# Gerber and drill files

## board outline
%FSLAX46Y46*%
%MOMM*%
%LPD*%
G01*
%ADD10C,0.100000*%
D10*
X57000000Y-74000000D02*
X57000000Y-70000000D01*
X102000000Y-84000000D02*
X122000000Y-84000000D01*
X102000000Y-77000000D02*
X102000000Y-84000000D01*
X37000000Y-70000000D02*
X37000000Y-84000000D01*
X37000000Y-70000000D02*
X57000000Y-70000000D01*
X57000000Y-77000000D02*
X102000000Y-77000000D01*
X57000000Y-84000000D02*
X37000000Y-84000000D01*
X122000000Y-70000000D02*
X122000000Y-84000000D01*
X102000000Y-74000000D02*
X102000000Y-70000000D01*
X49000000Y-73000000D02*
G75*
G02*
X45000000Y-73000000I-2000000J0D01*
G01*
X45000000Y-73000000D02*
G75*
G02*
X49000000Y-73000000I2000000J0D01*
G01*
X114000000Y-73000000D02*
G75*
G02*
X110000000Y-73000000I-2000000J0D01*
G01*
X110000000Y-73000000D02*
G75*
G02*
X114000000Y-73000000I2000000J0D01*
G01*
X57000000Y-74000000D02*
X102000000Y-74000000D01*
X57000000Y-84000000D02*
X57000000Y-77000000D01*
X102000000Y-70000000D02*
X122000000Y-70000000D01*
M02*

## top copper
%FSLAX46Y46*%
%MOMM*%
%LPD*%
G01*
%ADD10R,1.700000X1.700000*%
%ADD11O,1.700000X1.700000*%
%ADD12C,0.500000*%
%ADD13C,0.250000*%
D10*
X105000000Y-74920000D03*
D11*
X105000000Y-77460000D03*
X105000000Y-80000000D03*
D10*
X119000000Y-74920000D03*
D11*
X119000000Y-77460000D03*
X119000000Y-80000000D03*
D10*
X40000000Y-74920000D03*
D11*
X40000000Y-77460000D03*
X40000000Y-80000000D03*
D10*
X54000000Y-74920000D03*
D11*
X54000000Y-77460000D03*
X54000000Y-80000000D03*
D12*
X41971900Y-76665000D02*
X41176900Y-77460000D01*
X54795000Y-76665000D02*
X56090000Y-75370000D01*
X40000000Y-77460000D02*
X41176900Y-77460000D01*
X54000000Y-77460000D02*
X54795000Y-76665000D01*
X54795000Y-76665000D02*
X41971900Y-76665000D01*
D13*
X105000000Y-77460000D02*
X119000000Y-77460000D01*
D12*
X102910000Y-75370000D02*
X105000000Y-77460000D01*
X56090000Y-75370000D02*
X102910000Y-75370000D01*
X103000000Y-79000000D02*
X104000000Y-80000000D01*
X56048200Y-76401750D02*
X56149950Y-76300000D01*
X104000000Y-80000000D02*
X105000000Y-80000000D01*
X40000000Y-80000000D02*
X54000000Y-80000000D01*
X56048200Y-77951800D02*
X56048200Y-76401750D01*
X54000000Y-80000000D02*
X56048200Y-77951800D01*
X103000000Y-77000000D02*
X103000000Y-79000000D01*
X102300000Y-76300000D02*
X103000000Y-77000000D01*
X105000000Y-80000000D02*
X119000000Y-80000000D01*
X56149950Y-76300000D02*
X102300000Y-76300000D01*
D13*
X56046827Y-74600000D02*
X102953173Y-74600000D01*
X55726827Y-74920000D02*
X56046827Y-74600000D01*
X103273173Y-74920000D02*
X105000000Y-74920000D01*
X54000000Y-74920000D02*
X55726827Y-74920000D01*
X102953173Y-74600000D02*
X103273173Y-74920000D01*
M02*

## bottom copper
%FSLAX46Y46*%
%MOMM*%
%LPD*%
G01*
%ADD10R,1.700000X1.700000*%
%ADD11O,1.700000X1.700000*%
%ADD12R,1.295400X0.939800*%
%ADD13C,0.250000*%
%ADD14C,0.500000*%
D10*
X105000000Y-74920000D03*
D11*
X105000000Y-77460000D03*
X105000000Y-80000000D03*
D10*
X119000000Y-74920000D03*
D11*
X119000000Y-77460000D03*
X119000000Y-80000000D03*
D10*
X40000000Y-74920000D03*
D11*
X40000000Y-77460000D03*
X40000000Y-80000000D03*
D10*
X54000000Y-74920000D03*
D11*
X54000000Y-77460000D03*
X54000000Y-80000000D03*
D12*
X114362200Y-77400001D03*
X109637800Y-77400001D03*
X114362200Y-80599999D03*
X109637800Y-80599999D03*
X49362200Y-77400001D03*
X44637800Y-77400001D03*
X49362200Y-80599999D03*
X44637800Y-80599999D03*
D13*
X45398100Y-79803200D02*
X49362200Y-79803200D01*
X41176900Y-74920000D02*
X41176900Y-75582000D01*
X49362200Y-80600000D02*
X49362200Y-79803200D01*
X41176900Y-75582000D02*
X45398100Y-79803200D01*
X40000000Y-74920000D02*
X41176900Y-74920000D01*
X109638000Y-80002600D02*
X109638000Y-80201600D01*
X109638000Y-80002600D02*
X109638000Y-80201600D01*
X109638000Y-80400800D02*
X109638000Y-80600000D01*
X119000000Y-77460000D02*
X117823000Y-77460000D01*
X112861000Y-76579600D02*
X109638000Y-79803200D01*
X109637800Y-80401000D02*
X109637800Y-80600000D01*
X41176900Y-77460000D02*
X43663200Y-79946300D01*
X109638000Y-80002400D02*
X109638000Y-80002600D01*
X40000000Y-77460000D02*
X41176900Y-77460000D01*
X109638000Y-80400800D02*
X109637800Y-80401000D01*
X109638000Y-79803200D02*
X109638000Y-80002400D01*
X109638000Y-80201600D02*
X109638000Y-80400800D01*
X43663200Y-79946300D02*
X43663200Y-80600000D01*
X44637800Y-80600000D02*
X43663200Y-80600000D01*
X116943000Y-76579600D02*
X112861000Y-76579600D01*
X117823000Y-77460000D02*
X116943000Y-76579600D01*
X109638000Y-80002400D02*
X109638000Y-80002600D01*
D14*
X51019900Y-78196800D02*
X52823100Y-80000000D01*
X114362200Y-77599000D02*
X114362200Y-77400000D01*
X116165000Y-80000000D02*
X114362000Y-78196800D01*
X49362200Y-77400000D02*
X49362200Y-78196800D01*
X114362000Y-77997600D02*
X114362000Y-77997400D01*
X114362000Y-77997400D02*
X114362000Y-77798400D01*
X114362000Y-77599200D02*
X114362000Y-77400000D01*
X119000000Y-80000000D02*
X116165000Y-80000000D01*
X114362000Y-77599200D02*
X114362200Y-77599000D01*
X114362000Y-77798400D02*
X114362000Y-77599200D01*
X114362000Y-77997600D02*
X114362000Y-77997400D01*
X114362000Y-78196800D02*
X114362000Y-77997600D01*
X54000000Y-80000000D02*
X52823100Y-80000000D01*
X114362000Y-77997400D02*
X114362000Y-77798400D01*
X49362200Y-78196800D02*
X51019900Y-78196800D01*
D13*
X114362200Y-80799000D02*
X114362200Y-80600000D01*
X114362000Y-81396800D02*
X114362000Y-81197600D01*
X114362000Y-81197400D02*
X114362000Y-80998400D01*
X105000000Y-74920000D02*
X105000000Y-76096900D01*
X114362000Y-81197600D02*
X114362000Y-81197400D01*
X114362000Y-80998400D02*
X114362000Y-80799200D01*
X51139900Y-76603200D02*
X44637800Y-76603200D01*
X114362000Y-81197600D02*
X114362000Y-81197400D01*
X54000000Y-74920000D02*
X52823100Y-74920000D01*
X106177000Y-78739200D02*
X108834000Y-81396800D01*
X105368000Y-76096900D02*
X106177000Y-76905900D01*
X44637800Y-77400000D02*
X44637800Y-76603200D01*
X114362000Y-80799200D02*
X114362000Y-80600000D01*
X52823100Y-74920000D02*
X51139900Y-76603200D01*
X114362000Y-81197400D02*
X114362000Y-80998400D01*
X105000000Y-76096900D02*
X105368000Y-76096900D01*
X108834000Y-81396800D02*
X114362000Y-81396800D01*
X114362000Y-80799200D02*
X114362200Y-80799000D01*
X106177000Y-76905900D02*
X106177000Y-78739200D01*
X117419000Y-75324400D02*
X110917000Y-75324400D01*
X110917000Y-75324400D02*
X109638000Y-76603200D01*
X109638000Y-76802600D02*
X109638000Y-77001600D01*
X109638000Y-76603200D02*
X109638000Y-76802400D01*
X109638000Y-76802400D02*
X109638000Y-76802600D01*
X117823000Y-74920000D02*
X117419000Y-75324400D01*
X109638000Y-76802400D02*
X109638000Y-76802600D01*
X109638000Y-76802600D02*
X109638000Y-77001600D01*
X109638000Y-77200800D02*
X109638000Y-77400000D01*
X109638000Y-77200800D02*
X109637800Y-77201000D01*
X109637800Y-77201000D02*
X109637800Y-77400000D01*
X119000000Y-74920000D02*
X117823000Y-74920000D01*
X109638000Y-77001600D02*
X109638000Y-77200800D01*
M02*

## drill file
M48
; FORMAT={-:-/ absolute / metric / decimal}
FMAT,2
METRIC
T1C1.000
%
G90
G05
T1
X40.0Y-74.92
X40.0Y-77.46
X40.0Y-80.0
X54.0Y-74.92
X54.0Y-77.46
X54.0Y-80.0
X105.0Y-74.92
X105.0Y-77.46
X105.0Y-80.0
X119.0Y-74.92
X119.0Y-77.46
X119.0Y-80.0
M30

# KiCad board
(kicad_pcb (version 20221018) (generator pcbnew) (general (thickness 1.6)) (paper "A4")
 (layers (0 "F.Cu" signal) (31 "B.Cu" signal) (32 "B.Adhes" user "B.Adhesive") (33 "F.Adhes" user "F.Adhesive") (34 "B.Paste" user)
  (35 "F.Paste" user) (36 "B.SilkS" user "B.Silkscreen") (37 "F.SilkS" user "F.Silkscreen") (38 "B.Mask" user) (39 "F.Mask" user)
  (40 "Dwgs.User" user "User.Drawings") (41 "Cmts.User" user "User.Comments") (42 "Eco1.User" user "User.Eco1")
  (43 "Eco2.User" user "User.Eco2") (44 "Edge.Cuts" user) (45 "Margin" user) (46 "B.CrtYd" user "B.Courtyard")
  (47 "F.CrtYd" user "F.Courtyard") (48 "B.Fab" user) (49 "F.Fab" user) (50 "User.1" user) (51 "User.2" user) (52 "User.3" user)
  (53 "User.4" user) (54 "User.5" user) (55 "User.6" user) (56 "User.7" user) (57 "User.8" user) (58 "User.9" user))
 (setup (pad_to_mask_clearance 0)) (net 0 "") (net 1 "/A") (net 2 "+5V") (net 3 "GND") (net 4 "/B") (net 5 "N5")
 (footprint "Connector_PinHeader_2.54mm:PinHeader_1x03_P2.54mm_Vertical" (layer "F.Cu") (at 105 74.92)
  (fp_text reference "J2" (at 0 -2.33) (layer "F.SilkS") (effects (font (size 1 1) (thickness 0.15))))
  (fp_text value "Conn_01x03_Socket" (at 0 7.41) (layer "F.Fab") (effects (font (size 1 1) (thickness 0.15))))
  (pad "1" thru_hole rect (at 0 0) (size 1.7 1.7) (drill 1) (layers "*.Cu" "*.Mask") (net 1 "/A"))
  (pad "2" thru_hole oval (at 0 2.54) (size 1.7 1.7) (drill 1) (layers "*.Cu" "*.Mask") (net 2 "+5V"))
  (pad "3" thru_hole oval (at 0 5.08) (size 1.7 1.7) (drill 1) (layers "*.Cu" "*.Mask") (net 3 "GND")))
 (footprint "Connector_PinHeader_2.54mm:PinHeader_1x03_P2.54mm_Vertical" (layer "F.Cu") (at 119 74.92)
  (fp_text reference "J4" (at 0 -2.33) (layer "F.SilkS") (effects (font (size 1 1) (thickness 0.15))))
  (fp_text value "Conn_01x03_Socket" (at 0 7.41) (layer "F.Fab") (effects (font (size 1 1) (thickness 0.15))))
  (pad "1" thru_hole rect (at 0 0) (size 1.7 1.7) (drill 1) (layers "*.Cu" "*.Mask") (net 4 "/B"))
  (pad "2" thru_hole oval (at 0 2.54) (size 1.7 1.7) (drill 1) (layers "*.Cu" "*.Mask") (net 2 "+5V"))
  (pad "3" thru_hole oval (at 0 5.08) (size 1.7 1.7) (drill 1) (layers "*.Cu" "*.Mask") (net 3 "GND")))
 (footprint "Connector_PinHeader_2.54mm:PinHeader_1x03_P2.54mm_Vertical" (layer "F.Cu") (at 40 74.92)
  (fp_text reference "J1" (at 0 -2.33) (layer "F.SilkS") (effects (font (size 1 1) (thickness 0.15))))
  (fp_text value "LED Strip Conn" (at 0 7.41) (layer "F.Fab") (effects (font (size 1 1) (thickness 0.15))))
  (pad "1" thru_hole rect (at 0 0) (size 1.7 1.7) (drill 1) (layers "*.Cu" "*.Mask") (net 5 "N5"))
  (pad "2" thru_hole oval (at 0 2.54) (size 1.7 1.7) (drill 1) (layers "*.Cu" "*.Mask") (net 2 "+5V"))
  (pad "3" thru_hole oval (at 0 5.08) (size 1.7 1.7) (drill 1) (layers "*.Cu" "*.Mask") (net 3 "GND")))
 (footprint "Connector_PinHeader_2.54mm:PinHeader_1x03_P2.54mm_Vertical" (layer "F.Cu") (at 54 74.92)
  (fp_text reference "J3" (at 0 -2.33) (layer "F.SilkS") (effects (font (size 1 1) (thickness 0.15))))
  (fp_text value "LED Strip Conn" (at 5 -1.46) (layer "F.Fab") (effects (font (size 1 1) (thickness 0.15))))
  (pad "1" thru_hole rect (at 0 0) (size 1.7 1.7) (drill 1) (layers "*.Cu" "*.Mask") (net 1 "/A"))
  (pad "2" thru_hole oval (at 0 2.54) (size 1.7 1.7) (drill 1) (layers "*.Cu" "*.Mask") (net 2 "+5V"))
  (pad "3" thru_hole oval (at 0 5.08) (size 1.7 1.7) (drill 1) (layers "*.Cu" "*.Mask") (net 3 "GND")))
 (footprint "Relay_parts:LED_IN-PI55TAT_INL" (layer "B.Cu") (at 112 79 180)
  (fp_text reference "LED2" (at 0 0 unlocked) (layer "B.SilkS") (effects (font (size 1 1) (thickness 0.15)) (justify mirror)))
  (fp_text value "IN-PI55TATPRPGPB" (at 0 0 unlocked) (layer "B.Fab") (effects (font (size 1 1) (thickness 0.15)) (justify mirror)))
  (pad "1" smd rect (at -2.3622 1.599999 180) (size 1.2954 0.9398) (layers "B.Cu" "B.Paste" "B.Mask") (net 3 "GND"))
  (pad "2" smd rect (at 2.3622 1.599999 180) (size 1.2954 0.9398) (layers "B.Cu" "B.Paste" "B.Mask") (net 4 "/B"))
  (pad "3" smd rect (at -2.3622 -1.599999 180) (size 1.2954 0.9398) (layers "B.Cu" "B.Paste" "B.Mask") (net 1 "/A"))
  (pad "4" smd rect (at 2.3622 -1.599999 180) (size 1.2954 0.9398) (layers "B.Cu" "B.Paste" "B.Mask") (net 2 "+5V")))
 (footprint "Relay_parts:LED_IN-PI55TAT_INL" (layer "B.Cu") (at 47 79 180)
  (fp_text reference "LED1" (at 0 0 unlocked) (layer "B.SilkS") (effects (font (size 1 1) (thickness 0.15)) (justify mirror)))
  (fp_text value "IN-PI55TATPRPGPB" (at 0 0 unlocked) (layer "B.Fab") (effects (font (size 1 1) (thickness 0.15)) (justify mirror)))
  (pad "1" smd rect (at -2.3622 1.599999 180) (size 1.2954 0.9398) (layers "B.Cu" "B.Paste" "B.Mask") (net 3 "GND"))
  (pad "2" smd rect (at 2.3622 1.599999 180) (size 1.2954 0.9398) (layers "B.Cu" "B.Paste" "B.Mask") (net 1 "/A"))
  (pad "3" smd rect (at -2.3622 -1.599999 180) (size 1.2954 0.9398) (layers "B.Cu" "B.Paste" "B.Mask") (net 5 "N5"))
  (pad "4" smd rect (at 2.3622 -1.599999 180) (size 1.2954 0.9398) (layers "B.Cu" "B.Paste" "B.Mask") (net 2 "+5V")))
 (gr_line (start 57 74) (end 57 70) (stroke (width 0.1) (type default)) (layer "Edge.Cuts"))
 (gr_line (start 102 84) (end 122 84) (stroke (width 0.1) (type default)) (layer "Edge.Cuts"))
 (gr_line (start 102 77) (end 102 84) (stroke (width 0.1) (type default)) (layer "Edge.Cuts"))
 (gr_line (start 37 70) (end 37 84) (stroke (width 0.1) (type default)) (layer "Edge.Cuts"))
 (gr_line (start 37 70) (end 57 70) (stroke (width 0.1) (type default)) (layer "Edge.Cuts"))
 (gr_line (start 57 77) (end 102 77) (stroke (width 0.1) (type default)) (layer "Edge.Cuts"))
 (gr_line (start 57 84) (end 37 84) (stroke (width 0.1) (type default)) (layer "Edge.Cuts"))
 (gr_line (start 122 70) (end 122 84) (stroke (width 0.1) (type default)) (layer "Edge.Cuts"))
 (gr_line (start 102 74) (end 102 70) (stroke (width 0.1) (type default)) (layer "Edge.Cuts"))
 (gr_circle (center 47 73) (end 49 73) (stroke (width 0.1) (type default)) (fill none) (layer "Edge.Cuts"))
 (gr_circle (center 112 73) (end 110 73) (stroke (width 0.1) (type default)) (fill none) (layer "Edge.Cuts"))
 (gr_line (start 57 74) (end 102 74) (stroke (width 0.1) (type default)) (layer "Edge.Cuts"))
 (gr_line (start 57 84) (end 57 77) (stroke (width 0.1) (type default)) (layer "Edge.Cuts"))
 (gr_line (start 102 70) (end 122 70) (stroke (width 0.1) (type default)) (layer "Edge.Cuts"))
 (segment (start 45.3981 79.8032) (end 49.3622 79.8032) (width 0.25) (layer "B.Cu") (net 5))
 (segment (start 41.1769 74.92) (end 41.1769 75.582) (width 0.25) (layer "B.Cu") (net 5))
 (segment (start 49.3622 80.6) (end 49.3622 79.8032) (width 0.25) (layer "B.Cu") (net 5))
 (segment (start 41.1769 75.582) (end 45.3981 79.8032) (width 0.25) (layer "B.Cu") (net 5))
 (segment (start 40 74.92) (end 41.1769 74.92) (width 0.25) (layer "B.Cu") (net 5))
 (segment (start 41.9719 76.665) (end 41.1769 77.46) (width 0.5) (layer "F.Cu") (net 2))
 (segment (start 54.795 76.665) (end 56.09 75.37) (width 0.5) (layer "F.Cu") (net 2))
 (segment (start 40 77.46) (end 41.1769 77.46) (width 0.5) (layer "F.Cu") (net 2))
 (segment (start 54 77.46) (end 54.795 76.665) (width 0.5) (layer "F.Cu") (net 2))
 (segment (start 54.795 76.665) (end 41.9719 76.665) (width 0.5) (layer "F.Cu") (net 2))
 (segment (start 105 77.46) (end 119 77.46) (width 0.25) (layer "F.Cu") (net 2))
 (segment (start 102.91 75.37) (end 105 77.46) (width 0.5) (layer "F.Cu") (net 2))
 (segment (start 56.09 75.37) (end 102.91 75.37) (width 0.5) (layer "F.Cu") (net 2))
 (segment (start 109.638 80.0026) (end 109.638 80.2016) (width 0.25) (layer "B.Cu") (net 2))
 (segment (start 109.638 80.0026) (end 109.638 80.2016) (width 0.25) (layer "B.Cu") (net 2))
 (segment (start 109.638 80.4008) (end 109.638 80.6) (width 0.25) (layer "B.Cu") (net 2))
 (segment (start 119 77.46) (end 117.823 77.46) (width 0.25) (layer "B.Cu") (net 2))
 (segment (start 112.861 76.5796) (end 109.638 79.8032) (width 0.25) (layer "B.Cu") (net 2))
 (segment (start 109.6378 80.401) (end 109.6378 80.6) (width 0.25) (layer "B.Cu") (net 2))
 (segment (start 41.1769 77.46) (end 43.6632 79.9463) (width 0.25) (layer "B.Cu") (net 2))
 (segment (start 109.638 80.0024) (end 109.638 80.0026) (width 0.25) (layer "B.Cu") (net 2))
 (segment (start 40 77.46) (end 41.1769 77.46) (width 0.25) (layer "B.Cu") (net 2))
 (segment (start 109.638 80.4008) (end 109.6378 80.401) (width 0.25) (layer "B.Cu") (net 2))
 (segment (start 109.638 79.8032) (end 109.638 80.0024) (width 0.25) (layer "B.Cu") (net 2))
 (segment (start 109.638 80.2016) (end 109.638 80.4008) (width 0.25) (layer "B.Cu") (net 2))
 (segment (start 43.6632 79.9463) (end 43.6632 80.6) (width 0.25) (layer "B.Cu") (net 2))
 (segment (start 44.6378 80.6) (end 43.6632 80.6) (width 0.25) (layer "B.Cu") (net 2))
 (segment (start 116.943 76.5796) (end 112.861 76.5796) (width 0.25) (layer "B.Cu") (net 2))
 (segment (start 117.823 77.46) (end 116.943 76.5796) (width 0.25) (layer "B.Cu") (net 2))
 (segment (start 109.638 80.0024) (end 109.638 80.0026) (width 0.25) (layer "B.Cu") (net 2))
 (segment (start 103 79) (end 104 80) (width 0.5) (layer "F.Cu") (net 3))
 (segment (start 56.0482 76.40175) (end 56.14995 76.3) (width 0.5) (layer "F.Cu") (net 3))
 (segment (start 104 80) (end 105 80) (width 0.5) (layer "F.Cu") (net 3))
 (segment (start 40 80) (end 54 80) (width 0.5) (layer "F.Cu") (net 3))
 (segment (start 56.0482 77.9518) (end 56.0482 76.40175) (width 0.5) (layer "F.Cu") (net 3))
 (segment (start 54 80) (end 56.0482 77.9518) (width 0.5) (layer "F.Cu") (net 3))
 (segment (start 103 77) (end 103 79) (width 0.5) (layer "F.Cu") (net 3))
 (segment (start 102.3 76.3) (end 103 77) (width 0.5) (layer "F.Cu") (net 3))
 (segment (start 105 80) (end 119 80) (width 0.5) (layer "F.Cu") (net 3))
 (segment (start 56.14995 76.3) (end 102.3 76.3) (width 0.5) (layer "F.Cu") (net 3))
 (segment (start 51.0199 78.1968) (end 52.8231 80) (width 0.5) (layer "B.Cu") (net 3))
 (segment (start 114.3622 77.599) (end 114.3622 77.4) (width 0.5) (layer "B.Cu") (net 3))
 (segment (start 116.165 80) (end 114.362 78.1968) (width 0.5) (layer "B.Cu") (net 3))
 (segment (start 49.3622 77.4) (end 49.3622 78.1968) (width 0.5) (layer "B.Cu") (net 3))
 (segment (start 114.362 77.9976) (end 114.362 77.9974) (width 0.5) (layer "B.Cu") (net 3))
 (segment (start 114.362 77.9974) (end 114.362 77.7984) (width 0.5) (layer "B.Cu") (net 3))
 (segment (start 114.362 77.5992) (end 114.362 77.4) (width 0.5) (layer "B.Cu") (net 3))
 (segment (start 119 80) (end 116.165 80) (width 0.5) (layer "B.Cu") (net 3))
 (segment (start 114.362 77.5992) (end 114.3622 77.599) (width 0.5) (layer "B.Cu") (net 3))
 (segment (start 114.362 77.7984) (end 114.362 77.5992) (width 0.5) (layer "B.Cu") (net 3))
 (segment (start 114.362 77.9976) (end 114.362 77.9974) (width 0.5) (layer "B.Cu") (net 3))
 (segment (start 114.362 78.1968) (end 114.362 77.9976) (width 0.5) (layer "B.Cu") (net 3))
 (segment (start 54 80) (end 52.8231 80) (width 0.5) (layer "B.Cu") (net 3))
 (segment (start 114.362 77.9974) (end 114.362 77.7984) (width 0.5) (layer "B.Cu") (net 3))
 (segment (start 49.3622 78.1968) (end 51.0199 78.1968) (width 0.5) (layer "B.Cu") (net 3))
 (segment (start 56.046827 74.6) (end 102.953173 74.6) (width 0.25) (layer "F.Cu") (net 1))
 (segment (start 55.726827 74.92) (end 56.046827 74.6) (width 0.25) (layer "F.Cu") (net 1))
 (segment (start 103.273173 74.92) (end 105 74.92) (width 0.25) (layer "F.Cu") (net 1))
 (segment (start 54 74.92) (end 55.726827 74.92) (width 0.25) (layer "F.Cu") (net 1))
 (segment (start 102.953173 74.6) (end 103.273173 74.92) (width 0.25) (layer "F.Cu") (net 1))
 (segment (start 114.3622 80.799) (end 114.3622 80.6) (width 0.25) (layer "B.Cu") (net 1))
 (segment (start 114.362 81.3968) (end 114.362 81.1976) (width 0.25) (layer "B.Cu") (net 1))
 (segment (start 114.362 81.1974) (end 114.362 80.9984) (width 0.25) (layer "B.Cu") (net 1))
 (segment (start 105 74.92) (end 105 76.0969) (width 0.25) (layer "B.Cu") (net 1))
 (segment (start 114.362 81.1976) (end 114.362 81.1974) (width 0.25) (layer "B.Cu") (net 1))
 (segment (start 114.362 80.9984) (end 114.362 80.7992) (width 0.25) (layer "B.Cu") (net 1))
 (segment (start 51.1399 76.6032) (end 44.6378 76.6032) (width 0.25) (layer "B.Cu") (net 1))
 (segment (start 114.362 81.1976) (end 114.362 81.1974) (width 0.25) (layer "B.Cu") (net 1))
 (segment (start 54 74.92) (end 52.8231 74.92) (width 0.25) (layer "B.Cu") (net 1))
 (segment (start 106.177 78.7392) (end 108.834 81.3968) (width 0.25) (layer "B.Cu") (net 1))
 (segment (start 105.368 76.0969) (end 106.177 76.9059) (width 0.25) (layer "B.Cu") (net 1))
 (segment (start 44.6378 77.4) (end 44.6378 76.6032) (width 0.25) (layer "B.Cu") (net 1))
 (segment (start 114.362 80.7992) (end 114.362 80.6) (width 0.25) (layer "B.Cu") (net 1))
 (segment (start 52.8231 74.92) (end 51.1399 76.6032) (width 0.25) (layer "B.Cu") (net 1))
 (segment (start 114.362 81.1974) (end 114.362 80.9984) (width 0.25) (layer "B.Cu") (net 1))
 (segment (start 105 76.0969) (end 105.368 76.0969) (width 0.25) (layer "B.Cu") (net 1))
 (segment (start 108.834 81.3968) (end 114.362 81.3968) (width 0.25) (layer "B.Cu") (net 1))
 (segment (start 114.362 80.7992) (end 114.3622 80.799) (width 0.25) (layer "B.Cu") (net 1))
 (segment (start 106.177 76.9059) (end 106.177 78.7392) (width 0.25) (layer "B.Cu") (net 1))
 (segment (start 117.419 75.3244) (end 110.917 75.3244) (width 0.25) (layer "B.Cu") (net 4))
 (segment (start 110.917 75.3244) (end 109.638 76.6032) (width 0.25) (layer "B.Cu") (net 4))
 (segment (start 109.638 76.8026) (end 109.638 77.0016) (width 0.25) (layer "B.Cu") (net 4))
 (segment (start 109.638 76.6032) (end 109.638 76.8024) (width 0.25) (layer "B.Cu") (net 4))
 (segment (start 109.638 76.8024) (end 109.638 76.8026) (width 0.25) (layer "B.Cu") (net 4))
 (segment (start 117.823 74.92) (end 117.419 75.3244) (width 0.25) (layer "B.Cu") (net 4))
 (segment (start 109.638 76.8024) (end 109.638 76.8026) (width 0.25) (layer "B.Cu") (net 4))
 (segment (start 109.638 76.8026) (end 109.638 77.0016) (width 0.25) (layer "B.Cu") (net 4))
 (segment (start 109.638 77.2008) (end 109.638 77.4) (width 0.25) (layer "B.Cu") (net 4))
 (segment (start 109.638 77.2008) (end 109.6378 77.201) (width 0.25) (layer "B.Cu") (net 4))
 (segment (start 109.6378 77.201) (end 109.6378 77.4) (width 0.25) (layer "B.Cu") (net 4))
 (segment (start 119 74.92) (end 117.823 74.92) (width 0.25) (layer "B.Cu") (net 4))
 (segment (start 109.638 77.0016) (end 109.638 77.2008) (width 0.25) (layer "B.Cu") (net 4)))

